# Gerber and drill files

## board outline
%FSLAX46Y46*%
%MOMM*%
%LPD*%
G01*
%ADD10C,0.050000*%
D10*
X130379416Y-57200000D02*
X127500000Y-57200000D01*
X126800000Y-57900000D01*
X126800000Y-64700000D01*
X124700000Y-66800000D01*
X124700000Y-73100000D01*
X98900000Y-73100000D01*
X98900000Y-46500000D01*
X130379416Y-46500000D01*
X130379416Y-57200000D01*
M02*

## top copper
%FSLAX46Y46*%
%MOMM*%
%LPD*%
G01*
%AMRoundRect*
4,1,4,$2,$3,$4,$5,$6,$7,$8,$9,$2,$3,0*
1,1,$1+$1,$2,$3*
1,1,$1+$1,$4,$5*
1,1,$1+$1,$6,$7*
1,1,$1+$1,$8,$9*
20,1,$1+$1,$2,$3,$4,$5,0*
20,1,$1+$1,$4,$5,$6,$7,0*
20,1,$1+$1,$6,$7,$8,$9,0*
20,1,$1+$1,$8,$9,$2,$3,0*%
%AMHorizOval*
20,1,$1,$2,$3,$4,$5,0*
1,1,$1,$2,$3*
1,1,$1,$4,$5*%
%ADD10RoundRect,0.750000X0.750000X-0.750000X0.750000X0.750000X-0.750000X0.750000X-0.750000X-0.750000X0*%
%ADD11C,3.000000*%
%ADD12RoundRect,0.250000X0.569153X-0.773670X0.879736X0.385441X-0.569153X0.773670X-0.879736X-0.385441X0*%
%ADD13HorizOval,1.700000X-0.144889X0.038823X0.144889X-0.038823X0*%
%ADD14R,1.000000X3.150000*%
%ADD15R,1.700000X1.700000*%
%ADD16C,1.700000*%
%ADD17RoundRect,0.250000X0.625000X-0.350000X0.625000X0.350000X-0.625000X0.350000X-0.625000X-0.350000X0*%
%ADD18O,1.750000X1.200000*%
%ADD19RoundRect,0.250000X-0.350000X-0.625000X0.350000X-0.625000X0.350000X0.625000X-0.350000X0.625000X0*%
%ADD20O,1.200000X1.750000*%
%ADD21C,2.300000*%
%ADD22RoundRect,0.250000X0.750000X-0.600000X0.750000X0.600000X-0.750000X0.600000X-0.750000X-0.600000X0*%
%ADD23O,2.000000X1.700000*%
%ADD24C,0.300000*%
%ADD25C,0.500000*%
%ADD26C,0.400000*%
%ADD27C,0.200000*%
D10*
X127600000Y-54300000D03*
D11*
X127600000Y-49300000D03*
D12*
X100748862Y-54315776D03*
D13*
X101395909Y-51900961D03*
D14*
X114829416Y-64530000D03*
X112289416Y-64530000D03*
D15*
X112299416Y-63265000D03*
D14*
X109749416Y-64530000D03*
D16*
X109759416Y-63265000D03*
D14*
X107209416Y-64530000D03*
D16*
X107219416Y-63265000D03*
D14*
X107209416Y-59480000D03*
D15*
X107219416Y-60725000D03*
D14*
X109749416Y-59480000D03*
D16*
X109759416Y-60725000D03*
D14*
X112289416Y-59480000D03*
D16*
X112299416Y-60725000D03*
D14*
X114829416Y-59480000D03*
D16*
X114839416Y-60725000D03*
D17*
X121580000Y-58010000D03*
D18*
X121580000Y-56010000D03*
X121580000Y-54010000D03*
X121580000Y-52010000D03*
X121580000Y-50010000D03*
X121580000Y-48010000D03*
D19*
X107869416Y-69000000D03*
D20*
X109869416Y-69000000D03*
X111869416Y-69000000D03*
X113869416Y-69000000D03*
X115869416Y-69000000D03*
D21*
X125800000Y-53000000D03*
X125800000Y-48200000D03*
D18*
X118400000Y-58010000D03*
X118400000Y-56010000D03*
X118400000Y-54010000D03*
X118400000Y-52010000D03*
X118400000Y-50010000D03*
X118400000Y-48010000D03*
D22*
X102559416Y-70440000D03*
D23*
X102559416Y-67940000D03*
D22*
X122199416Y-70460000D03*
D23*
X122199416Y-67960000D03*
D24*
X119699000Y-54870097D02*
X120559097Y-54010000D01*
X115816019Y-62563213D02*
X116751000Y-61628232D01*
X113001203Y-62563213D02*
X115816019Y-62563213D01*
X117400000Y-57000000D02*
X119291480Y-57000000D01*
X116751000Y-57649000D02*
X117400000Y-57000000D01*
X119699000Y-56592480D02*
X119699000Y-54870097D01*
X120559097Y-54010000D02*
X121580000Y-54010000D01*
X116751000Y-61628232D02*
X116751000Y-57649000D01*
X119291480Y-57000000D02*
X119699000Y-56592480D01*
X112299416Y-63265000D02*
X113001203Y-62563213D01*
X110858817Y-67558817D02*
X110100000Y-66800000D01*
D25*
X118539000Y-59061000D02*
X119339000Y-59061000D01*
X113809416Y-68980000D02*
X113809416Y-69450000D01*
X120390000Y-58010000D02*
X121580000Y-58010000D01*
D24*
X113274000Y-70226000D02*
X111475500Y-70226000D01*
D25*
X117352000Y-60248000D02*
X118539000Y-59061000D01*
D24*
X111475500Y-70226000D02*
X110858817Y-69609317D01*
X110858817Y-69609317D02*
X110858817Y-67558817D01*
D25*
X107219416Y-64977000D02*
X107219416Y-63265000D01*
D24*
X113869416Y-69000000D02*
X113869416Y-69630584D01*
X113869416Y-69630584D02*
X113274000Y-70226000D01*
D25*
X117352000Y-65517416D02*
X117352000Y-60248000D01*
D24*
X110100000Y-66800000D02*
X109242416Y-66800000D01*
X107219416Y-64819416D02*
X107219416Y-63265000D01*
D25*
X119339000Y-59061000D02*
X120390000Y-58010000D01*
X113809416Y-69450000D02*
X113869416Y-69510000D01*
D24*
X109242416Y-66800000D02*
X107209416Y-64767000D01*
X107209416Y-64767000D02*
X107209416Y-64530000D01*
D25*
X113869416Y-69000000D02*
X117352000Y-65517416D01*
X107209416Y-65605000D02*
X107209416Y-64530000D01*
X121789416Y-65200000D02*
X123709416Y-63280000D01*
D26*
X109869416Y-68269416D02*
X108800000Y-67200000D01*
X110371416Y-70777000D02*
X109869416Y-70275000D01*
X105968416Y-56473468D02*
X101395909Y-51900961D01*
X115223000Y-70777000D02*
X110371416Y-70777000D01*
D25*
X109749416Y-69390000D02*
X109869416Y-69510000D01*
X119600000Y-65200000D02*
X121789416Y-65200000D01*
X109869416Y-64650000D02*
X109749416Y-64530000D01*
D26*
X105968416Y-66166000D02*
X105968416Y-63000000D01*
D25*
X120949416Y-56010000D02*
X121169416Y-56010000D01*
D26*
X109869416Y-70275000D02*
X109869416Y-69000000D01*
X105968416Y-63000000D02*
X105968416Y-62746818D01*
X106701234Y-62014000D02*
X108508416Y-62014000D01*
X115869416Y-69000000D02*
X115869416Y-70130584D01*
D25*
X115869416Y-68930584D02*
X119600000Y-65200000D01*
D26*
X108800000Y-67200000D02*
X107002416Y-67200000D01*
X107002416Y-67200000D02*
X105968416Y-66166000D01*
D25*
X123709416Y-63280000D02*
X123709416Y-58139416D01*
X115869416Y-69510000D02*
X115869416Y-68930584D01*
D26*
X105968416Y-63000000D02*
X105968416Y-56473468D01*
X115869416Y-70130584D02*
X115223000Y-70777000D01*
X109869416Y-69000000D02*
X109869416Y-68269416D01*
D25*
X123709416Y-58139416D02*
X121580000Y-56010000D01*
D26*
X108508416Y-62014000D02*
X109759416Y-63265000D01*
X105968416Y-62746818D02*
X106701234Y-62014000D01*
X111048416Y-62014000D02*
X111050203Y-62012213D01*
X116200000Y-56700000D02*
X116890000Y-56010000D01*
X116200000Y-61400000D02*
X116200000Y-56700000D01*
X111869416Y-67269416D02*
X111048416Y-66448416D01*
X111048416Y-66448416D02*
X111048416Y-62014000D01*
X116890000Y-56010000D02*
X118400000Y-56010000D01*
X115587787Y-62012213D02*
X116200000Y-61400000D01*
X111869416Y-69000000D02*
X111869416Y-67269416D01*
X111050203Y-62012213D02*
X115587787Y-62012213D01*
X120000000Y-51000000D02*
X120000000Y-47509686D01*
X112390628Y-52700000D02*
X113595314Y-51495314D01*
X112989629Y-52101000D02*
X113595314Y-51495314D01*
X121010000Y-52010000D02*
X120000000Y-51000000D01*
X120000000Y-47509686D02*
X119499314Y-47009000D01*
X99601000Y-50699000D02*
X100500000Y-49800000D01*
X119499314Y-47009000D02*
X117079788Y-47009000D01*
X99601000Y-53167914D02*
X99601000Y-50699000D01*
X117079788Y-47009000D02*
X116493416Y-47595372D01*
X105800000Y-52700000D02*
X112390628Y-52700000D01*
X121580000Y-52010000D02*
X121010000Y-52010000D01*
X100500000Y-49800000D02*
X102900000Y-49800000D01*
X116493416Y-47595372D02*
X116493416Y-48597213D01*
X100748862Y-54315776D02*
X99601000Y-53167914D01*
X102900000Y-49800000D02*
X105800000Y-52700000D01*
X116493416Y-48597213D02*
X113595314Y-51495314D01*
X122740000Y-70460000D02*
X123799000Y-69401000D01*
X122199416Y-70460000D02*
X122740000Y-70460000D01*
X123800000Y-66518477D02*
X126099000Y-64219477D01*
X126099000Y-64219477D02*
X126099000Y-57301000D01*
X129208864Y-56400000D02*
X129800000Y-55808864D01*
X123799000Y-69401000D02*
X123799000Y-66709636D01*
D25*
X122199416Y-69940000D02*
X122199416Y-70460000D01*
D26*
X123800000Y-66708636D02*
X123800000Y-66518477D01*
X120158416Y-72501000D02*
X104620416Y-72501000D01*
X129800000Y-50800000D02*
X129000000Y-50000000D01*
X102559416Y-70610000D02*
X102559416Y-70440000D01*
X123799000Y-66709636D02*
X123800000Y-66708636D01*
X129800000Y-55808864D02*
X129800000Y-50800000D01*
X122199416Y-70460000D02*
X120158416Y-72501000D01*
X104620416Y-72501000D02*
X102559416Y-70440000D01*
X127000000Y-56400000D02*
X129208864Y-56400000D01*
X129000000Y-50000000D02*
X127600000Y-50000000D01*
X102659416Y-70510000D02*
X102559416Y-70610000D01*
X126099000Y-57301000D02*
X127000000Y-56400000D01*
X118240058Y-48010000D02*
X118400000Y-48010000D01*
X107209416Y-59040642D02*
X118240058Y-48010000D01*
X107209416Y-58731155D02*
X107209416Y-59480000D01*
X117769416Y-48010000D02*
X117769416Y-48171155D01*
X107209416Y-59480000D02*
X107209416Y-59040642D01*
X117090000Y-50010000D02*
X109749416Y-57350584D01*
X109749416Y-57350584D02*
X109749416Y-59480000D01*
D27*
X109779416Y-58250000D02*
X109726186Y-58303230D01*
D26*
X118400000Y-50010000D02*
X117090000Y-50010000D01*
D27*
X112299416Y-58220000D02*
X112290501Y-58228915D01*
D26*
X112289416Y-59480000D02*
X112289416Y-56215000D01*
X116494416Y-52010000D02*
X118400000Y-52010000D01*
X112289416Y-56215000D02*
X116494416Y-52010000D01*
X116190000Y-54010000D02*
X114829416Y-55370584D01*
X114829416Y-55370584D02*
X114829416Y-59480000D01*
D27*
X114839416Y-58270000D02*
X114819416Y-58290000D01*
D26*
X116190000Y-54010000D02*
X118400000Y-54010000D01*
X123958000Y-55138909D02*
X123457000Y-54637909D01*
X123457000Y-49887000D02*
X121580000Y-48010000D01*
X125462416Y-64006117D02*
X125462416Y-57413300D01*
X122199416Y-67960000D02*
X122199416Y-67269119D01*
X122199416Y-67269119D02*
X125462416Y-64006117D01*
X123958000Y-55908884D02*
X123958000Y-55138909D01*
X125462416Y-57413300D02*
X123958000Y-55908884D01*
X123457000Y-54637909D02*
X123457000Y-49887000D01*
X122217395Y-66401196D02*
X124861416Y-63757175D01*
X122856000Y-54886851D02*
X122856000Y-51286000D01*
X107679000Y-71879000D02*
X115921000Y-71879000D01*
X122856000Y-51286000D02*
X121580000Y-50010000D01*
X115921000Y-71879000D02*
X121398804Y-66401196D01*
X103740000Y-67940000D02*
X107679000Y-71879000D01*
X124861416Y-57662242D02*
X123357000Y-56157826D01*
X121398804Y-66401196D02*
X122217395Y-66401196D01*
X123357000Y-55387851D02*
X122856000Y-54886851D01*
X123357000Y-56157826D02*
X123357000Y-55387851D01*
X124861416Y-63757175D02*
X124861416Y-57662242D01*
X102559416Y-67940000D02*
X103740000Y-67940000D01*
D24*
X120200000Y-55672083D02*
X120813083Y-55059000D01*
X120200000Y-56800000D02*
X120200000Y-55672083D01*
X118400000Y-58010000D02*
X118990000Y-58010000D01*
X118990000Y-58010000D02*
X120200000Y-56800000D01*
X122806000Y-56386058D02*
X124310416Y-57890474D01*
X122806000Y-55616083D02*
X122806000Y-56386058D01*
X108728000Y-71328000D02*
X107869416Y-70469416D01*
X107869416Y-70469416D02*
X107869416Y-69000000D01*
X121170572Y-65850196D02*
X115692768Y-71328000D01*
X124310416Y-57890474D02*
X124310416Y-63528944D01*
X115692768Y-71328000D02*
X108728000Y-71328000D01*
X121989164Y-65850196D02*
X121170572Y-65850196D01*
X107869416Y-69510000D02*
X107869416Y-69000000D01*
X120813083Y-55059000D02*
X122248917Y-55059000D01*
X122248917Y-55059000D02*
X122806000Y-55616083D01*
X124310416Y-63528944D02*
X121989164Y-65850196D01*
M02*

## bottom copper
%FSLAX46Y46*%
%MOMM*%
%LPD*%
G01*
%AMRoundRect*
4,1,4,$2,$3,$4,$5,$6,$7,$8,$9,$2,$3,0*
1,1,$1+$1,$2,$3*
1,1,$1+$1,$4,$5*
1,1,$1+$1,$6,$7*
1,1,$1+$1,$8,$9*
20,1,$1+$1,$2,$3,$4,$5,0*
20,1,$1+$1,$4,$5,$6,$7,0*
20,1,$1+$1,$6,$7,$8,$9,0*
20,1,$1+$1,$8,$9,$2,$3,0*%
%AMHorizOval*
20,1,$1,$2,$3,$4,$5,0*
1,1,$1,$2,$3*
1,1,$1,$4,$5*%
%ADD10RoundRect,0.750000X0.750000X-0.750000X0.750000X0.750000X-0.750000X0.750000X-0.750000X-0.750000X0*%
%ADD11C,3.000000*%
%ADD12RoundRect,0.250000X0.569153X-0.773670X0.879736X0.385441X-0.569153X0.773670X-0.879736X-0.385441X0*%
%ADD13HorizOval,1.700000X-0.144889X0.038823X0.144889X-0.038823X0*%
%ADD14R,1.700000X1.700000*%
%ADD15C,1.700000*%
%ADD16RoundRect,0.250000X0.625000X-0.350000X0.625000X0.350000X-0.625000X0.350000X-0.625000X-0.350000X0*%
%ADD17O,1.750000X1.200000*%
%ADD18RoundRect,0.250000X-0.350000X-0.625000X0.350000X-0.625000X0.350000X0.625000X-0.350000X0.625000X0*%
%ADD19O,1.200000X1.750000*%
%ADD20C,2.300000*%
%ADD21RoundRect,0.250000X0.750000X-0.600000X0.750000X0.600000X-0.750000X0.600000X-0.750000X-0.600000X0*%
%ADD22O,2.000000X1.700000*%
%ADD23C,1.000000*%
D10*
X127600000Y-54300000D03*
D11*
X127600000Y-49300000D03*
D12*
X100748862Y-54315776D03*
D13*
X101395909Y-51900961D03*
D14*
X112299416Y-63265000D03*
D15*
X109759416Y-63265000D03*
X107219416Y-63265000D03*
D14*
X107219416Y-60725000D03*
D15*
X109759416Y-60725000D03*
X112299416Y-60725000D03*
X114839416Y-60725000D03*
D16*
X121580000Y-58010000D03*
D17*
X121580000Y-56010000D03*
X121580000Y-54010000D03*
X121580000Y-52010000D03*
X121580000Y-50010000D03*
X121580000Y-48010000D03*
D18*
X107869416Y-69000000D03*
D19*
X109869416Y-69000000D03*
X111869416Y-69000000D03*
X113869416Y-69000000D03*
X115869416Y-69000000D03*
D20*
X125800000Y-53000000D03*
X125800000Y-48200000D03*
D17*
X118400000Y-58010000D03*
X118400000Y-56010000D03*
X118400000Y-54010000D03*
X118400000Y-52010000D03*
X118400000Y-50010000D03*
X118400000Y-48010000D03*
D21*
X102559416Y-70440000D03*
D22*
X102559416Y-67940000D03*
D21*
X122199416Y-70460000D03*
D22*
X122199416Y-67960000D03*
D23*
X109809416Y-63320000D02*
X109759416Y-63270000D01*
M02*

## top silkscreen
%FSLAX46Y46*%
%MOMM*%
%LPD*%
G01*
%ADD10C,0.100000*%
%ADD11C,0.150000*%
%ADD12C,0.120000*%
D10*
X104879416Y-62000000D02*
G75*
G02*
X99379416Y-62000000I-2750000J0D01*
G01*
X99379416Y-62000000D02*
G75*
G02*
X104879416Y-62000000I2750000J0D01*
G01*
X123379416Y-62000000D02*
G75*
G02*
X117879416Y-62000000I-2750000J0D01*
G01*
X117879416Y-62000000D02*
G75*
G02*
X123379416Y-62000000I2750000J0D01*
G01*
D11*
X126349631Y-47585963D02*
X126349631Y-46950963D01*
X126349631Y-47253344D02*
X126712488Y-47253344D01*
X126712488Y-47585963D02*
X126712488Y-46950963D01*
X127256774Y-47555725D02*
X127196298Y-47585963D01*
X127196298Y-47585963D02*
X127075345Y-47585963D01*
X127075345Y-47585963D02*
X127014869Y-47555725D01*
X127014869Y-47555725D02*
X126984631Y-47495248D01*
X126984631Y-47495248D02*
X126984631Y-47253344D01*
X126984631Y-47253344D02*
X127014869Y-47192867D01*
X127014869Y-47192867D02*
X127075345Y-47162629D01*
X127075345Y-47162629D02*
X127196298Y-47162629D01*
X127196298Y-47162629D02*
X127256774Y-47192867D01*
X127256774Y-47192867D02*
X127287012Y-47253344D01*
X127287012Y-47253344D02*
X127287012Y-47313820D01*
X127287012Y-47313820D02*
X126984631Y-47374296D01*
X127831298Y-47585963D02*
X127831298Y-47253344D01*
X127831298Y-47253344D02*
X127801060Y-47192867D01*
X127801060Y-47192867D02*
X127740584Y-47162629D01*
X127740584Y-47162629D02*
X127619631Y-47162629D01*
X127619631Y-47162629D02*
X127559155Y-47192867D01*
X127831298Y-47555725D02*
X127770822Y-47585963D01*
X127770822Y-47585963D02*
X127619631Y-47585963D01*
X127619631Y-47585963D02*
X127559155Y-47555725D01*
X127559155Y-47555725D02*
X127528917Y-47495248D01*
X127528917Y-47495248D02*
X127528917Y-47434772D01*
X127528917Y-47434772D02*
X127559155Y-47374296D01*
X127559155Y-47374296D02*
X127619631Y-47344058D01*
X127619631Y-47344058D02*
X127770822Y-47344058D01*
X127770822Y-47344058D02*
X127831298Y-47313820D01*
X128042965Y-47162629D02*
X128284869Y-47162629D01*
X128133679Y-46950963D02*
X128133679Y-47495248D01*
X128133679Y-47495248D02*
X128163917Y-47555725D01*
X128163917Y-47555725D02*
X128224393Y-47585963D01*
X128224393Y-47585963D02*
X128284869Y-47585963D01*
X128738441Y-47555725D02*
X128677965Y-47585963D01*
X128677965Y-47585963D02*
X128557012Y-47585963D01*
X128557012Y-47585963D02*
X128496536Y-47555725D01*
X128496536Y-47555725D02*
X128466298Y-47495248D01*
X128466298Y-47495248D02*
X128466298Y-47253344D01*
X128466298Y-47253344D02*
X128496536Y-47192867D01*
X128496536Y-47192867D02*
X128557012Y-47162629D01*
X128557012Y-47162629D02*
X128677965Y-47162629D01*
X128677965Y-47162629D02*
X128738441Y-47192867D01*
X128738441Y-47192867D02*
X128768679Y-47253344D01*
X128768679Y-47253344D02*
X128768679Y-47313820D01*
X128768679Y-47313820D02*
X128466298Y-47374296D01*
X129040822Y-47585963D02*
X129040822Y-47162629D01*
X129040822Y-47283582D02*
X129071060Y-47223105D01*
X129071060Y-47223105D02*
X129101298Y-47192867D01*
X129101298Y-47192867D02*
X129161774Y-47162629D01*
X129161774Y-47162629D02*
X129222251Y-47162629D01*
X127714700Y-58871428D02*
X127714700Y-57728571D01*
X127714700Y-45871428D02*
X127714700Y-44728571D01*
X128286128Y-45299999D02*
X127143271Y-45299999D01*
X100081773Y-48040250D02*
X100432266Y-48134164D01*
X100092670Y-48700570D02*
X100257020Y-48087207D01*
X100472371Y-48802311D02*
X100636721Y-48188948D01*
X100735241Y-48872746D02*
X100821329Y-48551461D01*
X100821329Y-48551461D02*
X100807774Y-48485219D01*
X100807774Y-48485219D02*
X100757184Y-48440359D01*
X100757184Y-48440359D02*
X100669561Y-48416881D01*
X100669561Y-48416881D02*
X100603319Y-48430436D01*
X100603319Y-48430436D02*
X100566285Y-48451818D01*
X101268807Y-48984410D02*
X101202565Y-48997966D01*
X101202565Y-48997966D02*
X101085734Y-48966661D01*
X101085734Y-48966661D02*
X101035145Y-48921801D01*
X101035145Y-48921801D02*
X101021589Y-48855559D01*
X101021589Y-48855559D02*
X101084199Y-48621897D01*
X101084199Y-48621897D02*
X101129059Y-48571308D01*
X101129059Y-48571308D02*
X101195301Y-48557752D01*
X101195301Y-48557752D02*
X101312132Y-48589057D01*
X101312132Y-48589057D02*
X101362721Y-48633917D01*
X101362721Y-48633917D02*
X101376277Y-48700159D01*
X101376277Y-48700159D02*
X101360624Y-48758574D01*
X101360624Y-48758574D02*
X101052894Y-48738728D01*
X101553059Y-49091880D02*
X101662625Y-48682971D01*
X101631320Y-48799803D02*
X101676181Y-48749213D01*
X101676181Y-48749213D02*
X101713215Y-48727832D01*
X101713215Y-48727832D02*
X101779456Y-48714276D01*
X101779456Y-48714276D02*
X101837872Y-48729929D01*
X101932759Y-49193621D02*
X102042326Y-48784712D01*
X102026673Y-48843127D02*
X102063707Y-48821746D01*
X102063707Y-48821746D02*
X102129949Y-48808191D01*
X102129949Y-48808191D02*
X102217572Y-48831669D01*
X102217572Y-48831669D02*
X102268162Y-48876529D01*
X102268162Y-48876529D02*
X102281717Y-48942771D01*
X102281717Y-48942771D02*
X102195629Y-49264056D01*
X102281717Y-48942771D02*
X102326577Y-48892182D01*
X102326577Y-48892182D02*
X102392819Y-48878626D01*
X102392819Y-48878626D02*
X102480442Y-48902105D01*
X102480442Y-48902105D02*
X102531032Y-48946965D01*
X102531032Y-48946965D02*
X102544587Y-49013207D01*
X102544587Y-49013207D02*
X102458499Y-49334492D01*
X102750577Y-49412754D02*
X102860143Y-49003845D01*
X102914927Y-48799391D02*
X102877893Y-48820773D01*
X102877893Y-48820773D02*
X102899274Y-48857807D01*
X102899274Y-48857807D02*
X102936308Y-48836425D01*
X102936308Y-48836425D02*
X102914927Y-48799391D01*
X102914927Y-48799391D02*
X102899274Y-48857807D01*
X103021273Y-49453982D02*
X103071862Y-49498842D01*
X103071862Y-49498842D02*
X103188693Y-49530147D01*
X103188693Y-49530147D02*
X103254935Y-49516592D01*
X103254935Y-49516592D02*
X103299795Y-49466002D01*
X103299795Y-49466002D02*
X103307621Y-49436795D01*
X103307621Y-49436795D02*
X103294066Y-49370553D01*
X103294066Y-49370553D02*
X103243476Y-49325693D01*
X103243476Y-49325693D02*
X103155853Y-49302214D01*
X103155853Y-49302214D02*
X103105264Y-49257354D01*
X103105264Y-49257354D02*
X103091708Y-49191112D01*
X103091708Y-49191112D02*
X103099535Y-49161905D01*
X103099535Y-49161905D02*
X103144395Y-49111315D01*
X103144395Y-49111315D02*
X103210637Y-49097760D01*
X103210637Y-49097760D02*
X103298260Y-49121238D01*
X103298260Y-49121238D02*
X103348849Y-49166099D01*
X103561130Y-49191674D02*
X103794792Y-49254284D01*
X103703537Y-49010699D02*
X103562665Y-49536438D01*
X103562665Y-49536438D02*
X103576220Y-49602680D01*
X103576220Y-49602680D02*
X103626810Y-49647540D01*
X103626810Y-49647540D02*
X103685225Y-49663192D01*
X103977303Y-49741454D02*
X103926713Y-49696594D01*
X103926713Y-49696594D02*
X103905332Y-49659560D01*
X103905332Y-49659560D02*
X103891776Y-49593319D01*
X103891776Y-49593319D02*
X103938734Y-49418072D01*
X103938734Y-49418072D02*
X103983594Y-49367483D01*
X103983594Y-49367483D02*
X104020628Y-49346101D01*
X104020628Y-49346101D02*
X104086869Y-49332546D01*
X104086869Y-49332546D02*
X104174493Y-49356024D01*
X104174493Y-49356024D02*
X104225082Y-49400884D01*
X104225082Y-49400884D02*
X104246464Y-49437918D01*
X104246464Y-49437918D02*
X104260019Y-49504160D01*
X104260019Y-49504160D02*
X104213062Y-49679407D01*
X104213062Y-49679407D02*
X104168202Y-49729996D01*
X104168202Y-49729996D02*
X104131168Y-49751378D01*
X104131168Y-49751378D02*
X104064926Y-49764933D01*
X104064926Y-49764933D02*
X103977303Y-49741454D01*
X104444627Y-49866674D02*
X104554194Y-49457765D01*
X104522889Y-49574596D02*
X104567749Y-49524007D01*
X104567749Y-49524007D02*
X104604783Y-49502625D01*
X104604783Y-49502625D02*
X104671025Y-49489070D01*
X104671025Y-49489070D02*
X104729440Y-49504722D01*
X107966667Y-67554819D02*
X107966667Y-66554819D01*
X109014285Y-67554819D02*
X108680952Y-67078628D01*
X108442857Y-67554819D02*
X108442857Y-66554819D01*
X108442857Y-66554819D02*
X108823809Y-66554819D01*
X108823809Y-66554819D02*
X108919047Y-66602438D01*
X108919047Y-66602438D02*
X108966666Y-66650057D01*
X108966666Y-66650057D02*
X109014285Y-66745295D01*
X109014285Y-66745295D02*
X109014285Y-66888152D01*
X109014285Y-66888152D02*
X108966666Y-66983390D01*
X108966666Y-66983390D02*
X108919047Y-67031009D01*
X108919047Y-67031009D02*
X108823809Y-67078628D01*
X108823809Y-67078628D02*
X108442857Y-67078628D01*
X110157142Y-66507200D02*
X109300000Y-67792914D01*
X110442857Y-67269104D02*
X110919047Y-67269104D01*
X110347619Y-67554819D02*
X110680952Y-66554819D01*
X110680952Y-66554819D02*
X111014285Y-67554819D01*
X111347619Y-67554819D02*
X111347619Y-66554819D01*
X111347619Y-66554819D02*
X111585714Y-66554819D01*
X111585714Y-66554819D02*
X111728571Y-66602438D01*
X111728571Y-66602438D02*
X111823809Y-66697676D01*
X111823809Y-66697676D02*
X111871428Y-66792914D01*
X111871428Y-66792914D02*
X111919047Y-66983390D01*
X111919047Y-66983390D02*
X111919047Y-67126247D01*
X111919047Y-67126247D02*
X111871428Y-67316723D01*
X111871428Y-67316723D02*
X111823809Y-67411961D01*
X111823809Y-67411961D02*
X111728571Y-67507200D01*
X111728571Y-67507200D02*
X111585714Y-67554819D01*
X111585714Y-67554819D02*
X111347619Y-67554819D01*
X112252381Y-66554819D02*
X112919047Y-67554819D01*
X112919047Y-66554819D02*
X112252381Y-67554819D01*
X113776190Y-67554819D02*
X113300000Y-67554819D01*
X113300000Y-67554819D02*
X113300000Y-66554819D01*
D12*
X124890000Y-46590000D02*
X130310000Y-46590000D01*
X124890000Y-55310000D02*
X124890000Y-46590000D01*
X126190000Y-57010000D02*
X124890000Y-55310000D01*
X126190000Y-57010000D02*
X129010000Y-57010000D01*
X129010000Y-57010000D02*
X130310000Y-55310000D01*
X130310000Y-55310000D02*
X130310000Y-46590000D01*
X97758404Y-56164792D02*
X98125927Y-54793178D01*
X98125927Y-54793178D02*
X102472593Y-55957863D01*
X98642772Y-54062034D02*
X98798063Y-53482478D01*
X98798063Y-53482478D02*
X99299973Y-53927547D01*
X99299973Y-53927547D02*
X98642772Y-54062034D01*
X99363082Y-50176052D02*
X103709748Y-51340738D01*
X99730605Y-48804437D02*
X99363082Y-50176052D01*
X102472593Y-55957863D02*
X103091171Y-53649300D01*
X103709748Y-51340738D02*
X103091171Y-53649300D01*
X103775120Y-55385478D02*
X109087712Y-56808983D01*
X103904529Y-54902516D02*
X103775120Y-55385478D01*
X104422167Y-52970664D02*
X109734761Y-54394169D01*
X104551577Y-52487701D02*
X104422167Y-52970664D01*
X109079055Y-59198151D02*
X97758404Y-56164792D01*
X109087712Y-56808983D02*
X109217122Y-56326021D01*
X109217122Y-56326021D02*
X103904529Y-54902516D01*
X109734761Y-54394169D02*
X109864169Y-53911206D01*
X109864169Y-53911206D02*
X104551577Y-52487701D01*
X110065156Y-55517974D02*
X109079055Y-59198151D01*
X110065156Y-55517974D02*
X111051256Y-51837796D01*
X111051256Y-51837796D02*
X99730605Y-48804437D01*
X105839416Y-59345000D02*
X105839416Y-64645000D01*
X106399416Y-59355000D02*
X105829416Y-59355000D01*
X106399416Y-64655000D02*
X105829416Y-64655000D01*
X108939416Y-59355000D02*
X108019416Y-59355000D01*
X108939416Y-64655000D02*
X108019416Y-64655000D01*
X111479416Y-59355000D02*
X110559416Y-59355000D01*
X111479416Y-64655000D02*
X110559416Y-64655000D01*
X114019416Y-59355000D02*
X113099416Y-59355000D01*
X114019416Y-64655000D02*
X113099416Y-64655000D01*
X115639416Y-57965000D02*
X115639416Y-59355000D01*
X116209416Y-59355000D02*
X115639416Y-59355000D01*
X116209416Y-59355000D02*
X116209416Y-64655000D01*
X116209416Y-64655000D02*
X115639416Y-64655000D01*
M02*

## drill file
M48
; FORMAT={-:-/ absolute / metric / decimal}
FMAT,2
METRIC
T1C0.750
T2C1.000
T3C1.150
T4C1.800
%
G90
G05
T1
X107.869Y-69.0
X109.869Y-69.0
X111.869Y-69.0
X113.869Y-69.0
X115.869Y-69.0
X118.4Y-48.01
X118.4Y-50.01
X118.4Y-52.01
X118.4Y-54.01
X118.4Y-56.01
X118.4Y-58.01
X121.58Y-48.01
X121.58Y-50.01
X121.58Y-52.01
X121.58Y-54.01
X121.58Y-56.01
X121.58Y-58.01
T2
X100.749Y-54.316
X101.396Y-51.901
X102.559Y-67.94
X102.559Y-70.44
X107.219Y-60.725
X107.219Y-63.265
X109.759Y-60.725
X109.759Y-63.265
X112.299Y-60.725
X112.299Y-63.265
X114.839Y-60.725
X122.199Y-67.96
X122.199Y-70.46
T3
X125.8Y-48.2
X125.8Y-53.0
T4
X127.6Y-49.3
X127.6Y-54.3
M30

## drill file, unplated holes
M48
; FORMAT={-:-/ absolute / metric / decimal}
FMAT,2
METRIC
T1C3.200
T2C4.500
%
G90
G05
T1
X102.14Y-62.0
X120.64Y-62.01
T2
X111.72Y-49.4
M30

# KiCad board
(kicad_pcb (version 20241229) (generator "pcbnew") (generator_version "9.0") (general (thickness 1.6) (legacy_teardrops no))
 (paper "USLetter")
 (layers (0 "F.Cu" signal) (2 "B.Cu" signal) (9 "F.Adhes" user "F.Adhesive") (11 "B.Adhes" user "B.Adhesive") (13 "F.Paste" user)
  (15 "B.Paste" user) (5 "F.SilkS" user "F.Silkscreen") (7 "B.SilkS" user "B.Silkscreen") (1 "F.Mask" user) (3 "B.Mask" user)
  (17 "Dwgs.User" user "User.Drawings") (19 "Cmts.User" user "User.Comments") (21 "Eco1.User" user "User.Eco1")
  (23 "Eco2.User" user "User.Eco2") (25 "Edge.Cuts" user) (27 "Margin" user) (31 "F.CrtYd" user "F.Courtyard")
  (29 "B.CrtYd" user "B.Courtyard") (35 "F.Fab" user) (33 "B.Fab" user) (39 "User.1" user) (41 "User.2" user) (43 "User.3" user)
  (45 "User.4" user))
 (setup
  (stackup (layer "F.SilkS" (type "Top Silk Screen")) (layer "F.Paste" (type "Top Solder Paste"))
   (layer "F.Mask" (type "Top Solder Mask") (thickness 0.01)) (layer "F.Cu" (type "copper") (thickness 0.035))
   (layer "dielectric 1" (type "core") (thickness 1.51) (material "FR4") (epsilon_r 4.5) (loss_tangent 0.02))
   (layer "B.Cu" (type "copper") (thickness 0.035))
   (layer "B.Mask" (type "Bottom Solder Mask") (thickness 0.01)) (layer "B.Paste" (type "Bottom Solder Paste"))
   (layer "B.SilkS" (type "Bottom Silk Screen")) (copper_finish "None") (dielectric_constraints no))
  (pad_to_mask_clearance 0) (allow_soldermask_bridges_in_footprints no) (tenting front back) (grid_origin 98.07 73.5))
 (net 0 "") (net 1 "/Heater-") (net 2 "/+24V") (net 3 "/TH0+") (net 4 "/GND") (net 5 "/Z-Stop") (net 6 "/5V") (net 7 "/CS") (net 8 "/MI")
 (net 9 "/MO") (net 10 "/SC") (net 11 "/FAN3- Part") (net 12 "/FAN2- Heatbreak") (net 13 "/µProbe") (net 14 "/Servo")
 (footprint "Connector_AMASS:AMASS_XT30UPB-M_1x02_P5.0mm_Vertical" (layer "F.Cu") (at 127.6 54.3 90)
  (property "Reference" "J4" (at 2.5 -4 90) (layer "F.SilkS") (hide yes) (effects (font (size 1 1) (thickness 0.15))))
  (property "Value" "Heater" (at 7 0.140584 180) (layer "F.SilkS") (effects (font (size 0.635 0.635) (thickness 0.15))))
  (fp_line (start 7.71 -2.71) (end 7.71 2.71) (stroke (width 0.12) (type solid)) (layer "F.SilkS"))
  (fp_line (start -1.01 -2.71) (end 7.71 -2.71) (stroke (width 0.12) (type solid)) (layer "F.SilkS"))
  (fp_line (start -2.71 -1.41) (end -1.01 -2.71) (stroke (width 0.12) (type solid)) (layer "F.SilkS"))
  (fp_line (start -2.71 -1.41) (end -2.71 1.41) (stroke (width 0.12) (type solid)) (layer "F.SilkS"))
  (fp_line (start -2.71 1.41) (end -1.01 2.71) (stroke (width 0.12) (type solid)) (layer "F.SilkS"))
  (fp_line (start -1.01 2.71) (end 7.71 2.71) (stroke (width 0.12) (type solid)) (layer "F.SilkS"))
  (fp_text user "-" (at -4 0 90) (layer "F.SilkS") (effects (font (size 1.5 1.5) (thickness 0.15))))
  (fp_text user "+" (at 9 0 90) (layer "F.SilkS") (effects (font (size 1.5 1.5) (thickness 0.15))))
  (pad "1" thru_hole roundrect (at 0 0 90) (size 3 3) (drill 1.8) (layers "*.Cu" "*.Mask") (remove_unused_layers no) (roundrect_rratio 0.25)
   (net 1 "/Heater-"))
  (pad "2" thru_hole circle (at 5 0 90) (size 3 3) (drill 1.8) (layers "*.Cu" "*.Mask") (remove_unused_layers no) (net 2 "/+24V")))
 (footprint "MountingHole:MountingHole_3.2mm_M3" (layer "F.Cu") (at 120.64 62.01)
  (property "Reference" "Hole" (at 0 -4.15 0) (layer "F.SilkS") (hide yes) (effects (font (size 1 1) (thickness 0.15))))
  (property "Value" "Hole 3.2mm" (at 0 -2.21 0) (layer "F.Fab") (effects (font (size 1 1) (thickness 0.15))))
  (pad "" np_thru_hole circle (at 0 0) (size 3.2 3.2) (drill 3.2) (layers "*.Cu" "*.Mask")))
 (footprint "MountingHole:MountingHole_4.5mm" (layer "F.Cu") (at 111.72 49.4)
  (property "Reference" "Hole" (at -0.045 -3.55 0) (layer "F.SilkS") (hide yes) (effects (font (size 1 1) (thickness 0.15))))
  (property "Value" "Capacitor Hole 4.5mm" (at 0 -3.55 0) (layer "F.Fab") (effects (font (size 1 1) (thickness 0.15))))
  (pad "" np_thru_hole circle (at 0 0) (size 4.5 4.5) (drill 4.5) (layers "*.Cu" "*.Mask")))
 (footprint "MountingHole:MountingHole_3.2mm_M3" (layer "F.Cu") (at 102.14 62)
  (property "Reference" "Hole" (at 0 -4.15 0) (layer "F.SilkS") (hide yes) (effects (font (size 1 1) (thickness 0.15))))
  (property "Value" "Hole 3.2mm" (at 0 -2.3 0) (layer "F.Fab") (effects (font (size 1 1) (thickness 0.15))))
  (pad "" np_thru_hole circle (at 0 0) (size 3.2 3.2) (drill 3.2) (layers "*.Cu" "*.Mask")))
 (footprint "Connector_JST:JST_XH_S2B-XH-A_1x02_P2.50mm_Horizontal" (layer "F.Cu") (at 100.748862 54.315776 75)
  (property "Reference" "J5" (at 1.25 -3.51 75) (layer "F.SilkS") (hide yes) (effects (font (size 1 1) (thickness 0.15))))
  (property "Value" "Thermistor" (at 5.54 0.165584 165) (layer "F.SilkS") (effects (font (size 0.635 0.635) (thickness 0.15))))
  (fp_line (start -2.56 -2.41) (end -1.14 -2.41) (stroke (width 0.12) (type solid)) (layer "F.SilkS"))
  (fp_line (start -1.14 -2.41) (end -1.14 2.09) (stroke (width 0.12) (type solid)) (layer "F.SilkS"))
  (fp_line (start -0.3 -2.1) (end 0.3 -2.100001) (stroke (width 0.12) (type solid)) (layer "F.SilkS"))
  (fp_line (start 0.3 -2.100001) (end 0 -1.5) (stroke (width 0.12) (type solid)) (layer "F.SilkS"))
  (fp_line (start 0 -1.5) (end -0.3 -2.1) (stroke (width 0.12) (type solid)) (layer "F.SilkS"))
  (fp_line (start 3.64 -2.41) (end 3.64 2.09) (stroke (width 0.12) (type solid)) (layer "F.SilkS"))
  (fp_line (start 5.06 -2.41) (end 3.64 -2.41) (stroke (width 0.12) (type solid)) (layer "F.SilkS"))
  (fp_line (start -1.14 2.09) (end 1.250001 2.09) (stroke (width 0.12) (type solid)) (layer "F.SilkS"))
  (fp_line (start 3.64 2.09) (end 1.250001 2.09) (stroke (width 0.12) (type solid)) (layer "F.SilkS"))
  (fp_line (start -0.25 3.2) (end -0.25 8.7) (stroke (width 0.12) (type solid)) (layer "F.SilkS"))
  (fp_line (start 0.249999 3.2) (end -0.25 3.2) (stroke (width 0.12) (type solid)) (layer "F.SilkS"))
  (fp_line (start 2.25 3.2) (end 2.25 8.700002) (stroke (width 0.12) (type solid)) (layer "F.SilkS"))
  (fp_line (start 2.75 3.2) (end 2.25 3.2) (stroke (width 0.12) (type solid)) (layer "F.SilkS"))
  (fp_line (start -2.56 9.31) (end -2.56 -2.41) (stroke (width 0.12) (type solid)) (layer "F.SilkS"))
  (fp_line (start -0.25 8.7) (end 0.249999 8.700001) (stroke (width 0.12) (type solid)) (layer "F.SilkS"))
  (fp_line (start 0.249999 8.700001) (end 0.249999 3.2) (stroke (width 0.12) (type solid)) (layer "F.SilkS"))
  (fp_line (start 2.25 8.700002) (end 2.75 8.7) (stroke (width 0.12) (type solid)) (layer "F.SilkS"))
  (fp_line (start 2.75 8.7) (end 2.75 3.2) (stroke (width 0.12) (type solid)) (layer "F.SilkS"))
  (fp_line (start 1.25 9.310001) (end -2.56 9.31) (stroke (width 0.12) (type solid)) (layer "F.SilkS"))
  (fp_line (start 1.25 9.310001) (end 5.060001 9.31) (stroke (width 0.12) (type solid)) (layer "F.SilkS"))
  (fp_line (start 5.060001 9.31) (end 5.06 -2.41) (stroke (width 0.12) (type solid)) (layer "F.SilkS"))
  (pad "1" thru_hole roundrect (at 0 0 75) (size 1.7 2) (drill 1) (layers "*.Cu" "*.Mask") (remove_unused_layers no)
   (roundrect_rratio 0.147059) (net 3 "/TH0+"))
  (pad "2" thru_hole oval (at 2.5 -0.000001 75) (size 1.7 2) (drill 1) (layers "*.Cu" "*.Mask") (remove_unused_layers no) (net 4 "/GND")))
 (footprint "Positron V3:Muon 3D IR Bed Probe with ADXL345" (layer "F.Cu") (at 109.339416 58.225)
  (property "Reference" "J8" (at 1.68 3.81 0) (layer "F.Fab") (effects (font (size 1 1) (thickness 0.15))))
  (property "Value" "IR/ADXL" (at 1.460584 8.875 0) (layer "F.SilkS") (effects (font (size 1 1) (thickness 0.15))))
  (fp_line (start -3.5 1.12) (end -3.5 6.42) (stroke (width 0.12) (type solid)) (layer "F.SilkS"))
  (fp_line (start -2.94 1.13) (end -3.51 1.13) (stroke (width 0.12) (type solid)) (layer "F.SilkS"))
  (fp_line (start -2.94 6.43) (end -3.51 6.43) (stroke (width 0.12) (type solid)) (layer "F.SilkS"))
  (fp_line (start -0.4 1.13) (end -1.32 1.13) (stroke (width 0.12) (type solid)) (layer "F.SilkS"))
  (fp_line (start -0.4 6.43) (end -1.32 6.43) (stroke (width 0.12) (type solid)) (layer "F.SilkS"))
  (fp_line (start 2.14 1.13) (end 1.22 1.13) (stroke (width 0.12) (type solid)) (layer "F.SilkS"))
  (fp_line (start 2.14 6.43) (end 1.22 6.43) (stroke (width 0.12) (type solid)) (layer "F.SilkS"))
  (fp_line (start 4.68 1.13) (end 3.76 1.13) (stroke (width 0.12) (type solid)) (layer "F.SilkS"))
  (fp_line (start 4.68 6.43) (end 3.76 6.43) (stroke (width 0.12) (type solid)) (layer "F.SilkS"))
  (fp_line (start 6.3 -0.26) (end 6.3 1.13) (stroke (width 0.12) (type solid)) (layer "F.SilkS"))
  (fp_line (start 6.87 1.13) (end 6.3 1.13) (stroke (width 0.12) (type solid)) (layer "F.SilkS"))
  (fp_line (start 6.87 1.13) (end 6.87 6.43) (stroke (width 0.12) (type solid)) (layer "F.SilkS"))
  (fp_line (start 6.87 6.43) (end 6.3 6.43) (stroke (width 0.12) (type solid)) (layer "F.SilkS"))
  (pad "" smd rect (at 5.49 6.305 270) (size 3.15 1) (layers "F.Cu" "F.Mask" "F.Paste"))
  (pad "1" smd rect (at 2.95 6.305 270) (size 3.15 1) (layers "F.Cu" "F.Mask" "F.Paste") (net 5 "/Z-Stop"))
  (pad "1" thru_hole rect (at 2.96 5.04 270) (size 1.7 1.7) (drill 1) (layers "*.Cu" "*.Mask") (remove_unused_layers no) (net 5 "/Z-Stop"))
  (pad "2" smd rect (at 0.41 6.305 270) (size 3.15 1) (layers "F.Cu" "F.Mask" "F.Paste") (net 4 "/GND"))
  (pad "2" thru_hole circle (at 0.42 5.04 270) (size 1.7 1.7) (drill 1) (layers "*.Cu" "*.Mask") (remove_unused_layers no) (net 4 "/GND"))
  (pad "3" smd rect (at -2.13 6.305 270) (size 3.15 1) (layers "F.Cu" "F.Mask" "F.Paste") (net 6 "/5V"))
  (pad "3" thru_hole circle (at -2.12 5.04 270) (size 1.7 1.7) (drill 1) (layers "*.Cu" "*.Mask") (remove_unused_layers no) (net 6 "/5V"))
  (pad "4" smd rect (at -2.13 1.255 270) (size 3.15 1) (layers "F.Cu" "F.Mask" "F.Paste") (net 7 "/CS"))
  (pad "4" thru_hole rect (at -2.12 2.5 270) (size 1.7 1.7) (drill 1) (layers "*.Cu" "*.Mask") (remove_unused_layers no) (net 7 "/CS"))
  (pad "5" smd rect (at 0.41 1.255 270) (size 3.15 1) (layers "F.Cu" "F.Mask" "F.Paste") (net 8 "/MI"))
  (pad "5" thru_hole circle (at 0.42 2.5 270) (size 1.7 1.7) (drill 1) (layers "*.Cu" "*.Mask") (remove_unused_layers no) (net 8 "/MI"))
  (pad "6" smd rect (at 2.95 1.255 270) (size 3.15 1) (layers "F.Cu" "F.Mask" "F.Paste") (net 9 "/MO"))
  (pad "6" thru_hole circle (at 2.96 2.5 270) (size 1.7 1.7) (drill 1) (layers "*.Cu" "*.Mask") (remove_unused_layers no) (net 9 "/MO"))
  (pad "7" smd rect (at 5.49 1.255 270) (size 3.15 1) (layers "F.Cu" "F.Mask" "F.Paste") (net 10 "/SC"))
  (pad "7" thru_hole circle (at 5.5 2.5 270) (size 1.7 1.7) (drill 1) (layers "*.Cu" "*.Mask") (remove_unused_layers no) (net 10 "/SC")))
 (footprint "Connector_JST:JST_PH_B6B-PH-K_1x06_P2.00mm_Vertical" (layer "B.Cu") (at 121.58 58.01 90)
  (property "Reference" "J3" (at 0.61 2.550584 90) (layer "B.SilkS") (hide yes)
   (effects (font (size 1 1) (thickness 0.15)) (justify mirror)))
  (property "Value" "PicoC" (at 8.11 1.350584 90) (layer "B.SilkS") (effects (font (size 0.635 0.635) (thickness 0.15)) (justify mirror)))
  (pad "1" thru_hole roundrect (at 0 0 90) (size 1.2 1.75) (drill 0.75) (layers "*.Cu" "*.Mask") (remove_unused_layers no)
   (roundrect_rratio 0.208333) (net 6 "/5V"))
  (pad "2" thru_hole oval (at 2 0 90) (size 1.2 1.75) (drill 0.75) (layers "*.Cu" "*.Mask") (remove_unused_layers no) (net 4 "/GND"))
  (pad "3" thru_hole oval (at 4 0 90) (size 1.2 1.75) (drill 0.75) (layers "*.Cu" "*.Mask") (remove_unused_layers no) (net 5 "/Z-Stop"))
  (pad "4" thru_hole oval (at 6 0 90) (size 1.2 1.75) (drill 0.75) (layers "*.Cu" "*.Mask") (remove_unused_layers no) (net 3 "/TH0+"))
  (pad "5" thru_hole oval (at 8 0 90) (size 1.2 1.75) (drill 0.75) (layers "*.Cu" "*.Mask") (remove_unused_layers no) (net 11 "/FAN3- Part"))
  (pad "6" thru_hole oval (at 10 0 90) (size 1.2 1.75) (drill 0.75) (layers "*.Cu" "*.Mask") (remove_unused_layers no)
   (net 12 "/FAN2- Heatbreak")))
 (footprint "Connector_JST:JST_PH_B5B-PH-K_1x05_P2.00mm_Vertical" (layer "B.Cu") (at 107.869416 69)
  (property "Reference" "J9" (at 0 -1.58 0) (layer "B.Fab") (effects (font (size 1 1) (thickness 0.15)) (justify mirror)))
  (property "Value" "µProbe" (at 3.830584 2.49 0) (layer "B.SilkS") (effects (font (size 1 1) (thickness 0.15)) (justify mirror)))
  (pad "1" thru_hole roundrect (at 0 0) (size 1.2 1.75) (drill 0.75) (layers "*.Cu" "*.Mask") (remove_unused_layers no)
   (roundrect_rratio 0.208333) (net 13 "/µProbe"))
  (pad "2" thru_hole oval (at 2 0) (size 1.2 1.75) (drill 0.75) (layers "*.Cu" "*.Mask") (remove_unused_layers no) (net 4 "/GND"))
  (pad "3" thru_hole oval (at 4 0) (size 1.2 1.75) (drill 0.75) (layers "*.Cu" "*.Mask") (remove_unused_layers no) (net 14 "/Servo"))
  (pad "4" thru_hole oval (at 6 0) (size 1.2 1.75) (drill 0.75) (layers "*.Cu" "*.Mask") (remove_unused_layers no) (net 6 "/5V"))
  (pad "5" thru_hole oval (at 8 0) (size 1.2 1.75) (drill 0.75) (layers "*.Cu" "*.Mask") (remove_unused_layers no) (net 4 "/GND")))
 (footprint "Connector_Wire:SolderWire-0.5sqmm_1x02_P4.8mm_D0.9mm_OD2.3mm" (layer "B.Cu") (at 125.8 53 90)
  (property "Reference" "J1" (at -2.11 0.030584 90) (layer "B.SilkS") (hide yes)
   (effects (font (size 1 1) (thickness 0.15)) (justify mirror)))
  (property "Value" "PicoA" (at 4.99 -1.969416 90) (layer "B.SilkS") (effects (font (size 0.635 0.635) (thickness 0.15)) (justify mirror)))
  (pad "1" thru_hole circle (at 0 0 90) (size 2.3 2.3) (drill 1.15) (layers "*.Cu" "*.Mask") (remove_unused_layers no) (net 1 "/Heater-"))
  (pad "2" thru_hole circle (at 4.8 0 90) (size 2.3 2.3) (drill 1.15) (layers "*.Cu" "*.Mask") (remove_unused_layers no) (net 2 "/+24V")))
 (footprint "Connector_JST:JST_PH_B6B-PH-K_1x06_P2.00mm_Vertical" (layer "B.Cu") (at 118.4 58.01 90)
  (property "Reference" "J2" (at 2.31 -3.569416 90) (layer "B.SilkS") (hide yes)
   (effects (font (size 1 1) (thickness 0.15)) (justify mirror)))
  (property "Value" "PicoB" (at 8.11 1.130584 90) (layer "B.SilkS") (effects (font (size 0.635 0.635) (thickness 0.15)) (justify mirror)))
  (pad "1" thru_hole oval (at 0 0 90) (size 1.2 1.75) (drill 0.75) (layers "*.Cu" "*.Mask") (remove_unused_layers no) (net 13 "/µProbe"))
  (pad "2" thru_hole oval (at 2 0 90) (size 1.2 1.75) (drill 0.75) (layers "*.Cu" "*.Mask") (remove_unused_layers no) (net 14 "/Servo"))
  (pad "3" thru_hole oval (at 4 0 90) (size 1.2 1.75) (drill 0.75) (layers "*.Cu" "*.Mask") (remove_unused_layers no) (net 10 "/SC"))
  (pad "4" thru_hole oval (at 6 0 90) (size 1.2 1.75) (drill 0.75) (layers "*.Cu" "*.Mask") (remove_unused_layers no) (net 9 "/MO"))
  (pad "5" thru_hole oval (at 8 0 90) (size 1.2 1.75) (drill 0.75) (layers "*.Cu" "*.Mask") (remove_unused_layers no) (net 8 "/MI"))
  (pad "6" thru_hole oval (at 10 0 90) (size 1.2 1.75) (drill 0.75) (layers "*.Cu" "*.Mask") (remove_unused_layers no) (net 7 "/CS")))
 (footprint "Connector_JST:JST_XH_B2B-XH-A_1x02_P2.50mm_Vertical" (layer "B.Cu") (at 102.559416 70.44 90)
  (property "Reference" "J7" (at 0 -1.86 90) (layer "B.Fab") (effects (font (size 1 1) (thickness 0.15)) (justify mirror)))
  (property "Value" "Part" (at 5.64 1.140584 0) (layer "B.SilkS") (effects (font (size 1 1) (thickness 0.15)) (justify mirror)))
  (pad "1" thru_hole roundrect (at 0 0 90) (size 1.7 2) (drill 1) (layers "*.Cu" "*.Mask") (remove_unused_layers no)
   (roundrect_rratio 0.147059) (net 2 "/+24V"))
  (pad "2" thru_hole oval (at 2.5 0 90) (size 1.7 2) (drill 1) (layers "*.Cu" "*.Mask") (remove_unused_layers no) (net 11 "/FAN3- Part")))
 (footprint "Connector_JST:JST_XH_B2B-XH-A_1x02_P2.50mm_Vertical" (layer "B.Cu") (at 122.199416 70.46 90)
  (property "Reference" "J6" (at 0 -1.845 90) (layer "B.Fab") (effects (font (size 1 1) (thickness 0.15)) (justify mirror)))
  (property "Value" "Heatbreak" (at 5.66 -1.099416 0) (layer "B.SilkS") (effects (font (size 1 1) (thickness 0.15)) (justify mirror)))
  (pad "1" thru_hole roundrect (at 0 0 90) (size 1.7 2) (drill 1) (layers "*.Cu" "*.Mask") (remove_unused_layers no)
   (roundrect_rratio 0.147059) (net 2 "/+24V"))
  (pad "2" thru_hole oval (at 2.5 0 90) (size 1.7 2) (drill 1) (layers "*.Cu" "*.Mask") (remove_unused_layers no)
   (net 12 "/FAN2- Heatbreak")))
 (gr_circle (center 102.129416 62) (end 104.879416 62) (stroke (width 0.1) (type solid)) (fill no) (layer "F.SilkS"))
 (gr_circle (center 120.629416 62) (end 123.379416 62) (stroke (width 0.1) (type solid)) (fill no) (layer "F.SilkS"))
 (gr_poly
  (pts (xy 130.379416 46.5) (xy 130.379416 57.2) (xy 127.5 57.2) (xy 126.8 57.9) (xy 126.8 64.7) (xy 124.7 66.8) (xy 124.7 73.1)
   (xy 98.9 73.1) (xy 98.9 46.5))
  (stroke (width 0.05) (type solid)) (fill no) (layer "Edge.Cuts"))
 (segment (start 119.699 54.870097) (end 120.559097 54.01) (width 0.3) (layer "F.Cu") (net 5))
 (segment (start 115.816019 62.563213) (end 116.751 61.628232) (width 0.3) (layer "F.Cu") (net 5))
 (segment (start 113.001203 62.563213) (end 115.816019 62.563213) (width 0.3) (layer "F.Cu") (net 5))
 (segment (start 117.4 57) (end 119.29148 57) (width 0.3) (layer "F.Cu") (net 5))
 (segment (start 116.751 57.649) (end 117.4 57) (width 0.3) (layer "F.Cu") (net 5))
 (segment (start 119.699 56.59248) (end 119.699 54.870097) (width 0.3) (layer "F.Cu") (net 5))
 (segment (start 120.559097 54.01) (end 121.58 54.01) (width 0.3) (layer "F.Cu") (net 5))
 (segment (start 116.751 61.628232) (end 116.751 57.649) (width 0.3) (layer "F.Cu") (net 5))
 (segment (start 119.29148 57) (end 119.699 56.59248) (width 0.3) (layer "F.Cu") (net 5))
 (segment (start 112.299416 63.265) (end 113.001203 62.563213) (width 0.3) (layer "F.Cu") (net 5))
 (segment (start 110.858817 67.558817) (end 110.1 66.8) (width 0.3) (layer "F.Cu") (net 6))
 (segment (start 118.539 59.061) (end 119.339 59.061) (width 0.5) (layer "F.Cu") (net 6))
 (segment (start 113.809416 68.98) (end 113.809416 69.45) (width 0.5) (layer "F.Cu") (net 6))
 (segment (start 120.39 58.01) (end 121.58 58.01) (width 0.5) (layer "F.Cu") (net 6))
 (segment (start 113.274 70.226) (end 111.4755 70.226) (width 0.3) (layer "F.Cu") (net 6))
 (segment (start 117.352 60.248) (end 118.539 59.061) (width 0.5) (layer "F.Cu") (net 6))
 (segment (start 111.4755 70.226) (end 110.858817 69.609317) (width 0.3) (layer "F.Cu") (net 6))
 (segment (start 110.858817 69.609317) (end 110.858817 67.558817) (width 0.3) (layer "F.Cu") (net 6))
 (segment (start 107.219416 64.977) (end 107.219416 63.265) (width 0.5) (layer "F.Cu") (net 6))
 (segment (start 113.869416 69) (end 113.869416 69.630584) (width 0.3) (layer "F.Cu") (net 6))
 (segment (start 113.869416 69.630584) (end 113.274 70.226) (width 0.3) (layer "F.Cu") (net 6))
 (segment (start 117.352 65.517416) (end 117.352 60.248) (width 0.5) (layer "F.Cu") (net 6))
 (segment (start 110.1 66.8) (end 109.242416 66.8) (width 0.3) (layer "F.Cu") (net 6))
 (segment (start 107.219416 64.819416) (end 107.219416 63.265) (width 0.3) (layer "F.Cu") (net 6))
 (segment (start 119.339 59.061) (end 120.39 58.01) (width 0.5) (layer "F.Cu") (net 6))
 (segment (start 113.809416 69.45) (end 113.869416 69.51) (width 0.5) (layer "F.Cu") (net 6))
 (segment (start 109.242416 66.8) (end 107.209416 64.767) (width 0.3) (layer "F.Cu") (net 6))
 (segment (start 107.209416 64.767) (end 107.209416 64.53) (width 0.3) (layer "F.Cu") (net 6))
 (segment (start 113.869416 69) (end 117.352 65.517416) (width 0.5) (layer "F.Cu") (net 6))
 (segment (start 107.209416 65.605) (end 107.209416 64.53) (width 0.5) (layer "F.Cu") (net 6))
 (segment (start 121.789416 65.2) (end 123.709416 63.28) (width 0.5) (layer "F.Cu") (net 4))
 (segment (start 109.869416 68.269416) (end 108.8 67.2) (width 0.4) (layer "F.Cu") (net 4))
 (segment (start 110.371416 70.777) (end 109.869416 70.275) (width 0.4) (layer "F.Cu") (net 4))
 (segment (start 105.968416 56.473468) (end 101.395909 51.900961) (width 0.4) (layer "F.Cu") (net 4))
 (segment (start 115.223 70.777) (end 110.371416 70.777) (width 0.4) (layer "F.Cu") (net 4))
 (segment (start 109.749416 69.39) (end 109.869416 69.51) (width 0.5) (layer "F.Cu") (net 4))
 (segment (start 119.6 65.2) (end 121.789416 65.2) (width 0.5) (layer "F.Cu") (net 4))
 (segment (start 109.869416 64.65) (end 109.749416 64.53) (width 0.5) (layer "F.Cu") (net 4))
 (segment (start 105.968416 66.166) (end 105.968416 63) (width 0.4) (layer "F.Cu") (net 4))
 (segment (start 120.949416 56.01) (end 121.169416 56.01) (width 0.5) (layer "F.Cu") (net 4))
 (segment (start 109.869416 70.275) (end 109.869416 69) (width 0.4) (layer "F.Cu") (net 4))
 (segment (start 105.968416 63) (end 105.968416 62.746818) (width 0.4) (layer "F.Cu") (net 4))
 (segment (start 106.701234 62.014) (end 108.508416 62.014) (width 0.4) (layer "F.Cu") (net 4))
 (segment (start 115.869416 69) (end 115.869416 70.130584) (width 0.4) (layer "F.Cu") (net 4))
 (segment (start 115.869416 68.930584) (end 119.6 65.2) (width 0.5) (layer "F.Cu") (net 4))
 (segment (start 108.8 67.2) (end 107.002416 67.2) (width 0.4) (layer "F.Cu") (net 4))
 (segment (start 107.002416 67.2) (end 105.968416 66.166) (width 0.4) (layer "F.Cu") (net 4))
 (segment (start 123.709416 63.28) (end 123.709416 58.139416) (width 0.5) (layer "F.Cu") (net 4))
 (segment (start 115.869416 69.51) (end 115.869416 68.930584) (width 0.5) (layer "F.Cu") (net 4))
 (segment (start 105.968416 63) (end 105.968416 56.473468) (width 0.4) (layer "F.Cu") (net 4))
 (segment (start 115.869416 70.130584) (end 115.223 70.777) (width 0.4) (layer "F.Cu") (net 4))
 (segment (start 109.869416 69) (end 109.869416 68.269416) (width 0.4) (layer "F.Cu") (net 4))
 (segment (start 123.709416 58.139416) (end 121.58 56.01) (width 0.5) (layer "F.Cu") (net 4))
 (segment (start 108.508416 62.014) (end 109.759416 63.265) (width 0.4) (layer "F.Cu") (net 4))
 (segment (start 105.968416 62.746818) (end 106.701234 62.014) (width 0.4) (layer "F.Cu") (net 4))
 (segment (start 109.809416 63.32) (end 109.759416 63.27) (width 1) (layer "B.Cu") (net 4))
 (segment (start 111.048416 62.014) (end 111.050203 62.012213) (width 0.4) (layer "F.Cu") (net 14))
 (segment (start 116.2 56.7) (end 116.89 56.01) (width 0.4) (layer "F.Cu") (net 14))
 (segment (start 116.2 61.4) (end 116.2 56.7) (width 0.4) (layer "F.Cu") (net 14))
 (segment (start 111.869416 67.269416) (end 111.048416 66.448416) (width 0.4) (layer "F.Cu") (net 14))
 (segment (start 111.048416 66.448416) (end 111.048416 62.014) (width 0.4) (layer "F.Cu") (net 14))
 (segment (start 116.89 56.01) (end 118.4 56.01) (width 0.4) (layer "F.Cu") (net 14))
 (segment (start 115.587787 62.012213) (end 116.2 61.4) (width 0.4) (layer "F.Cu") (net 14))
 (segment (start 111.869416 69) (end 111.869416 67.269416) (width 0.4) (layer "F.Cu") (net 14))
 (segment (start 111.050203 62.012213) (end 115.587787 62.012213) (width 0.4) (layer "F.Cu") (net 14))
 (segment (start 120 51) (end 120 47.509686) (width 0.4) (layer "F.Cu") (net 3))
 (segment (start 112.390628 52.7) (end 113.595314 51.495314) (width 0.4) (layer "F.Cu") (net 3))
 (segment (start 112.989629 52.101) (end 113.595314 51.495314) (width 0.4) (layer "F.Cu") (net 3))
 (segment (start 121.01 52.01) (end 120 51) (width 0.4) (layer "F.Cu") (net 3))
 (segment (start 120 47.509686) (end 119.499314 47.009) (width 0.4) (layer "F.Cu") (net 3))
 (segment (start 99.601 50.699) (end 100.5 49.8) (width 0.4) (layer "F.Cu") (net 3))
 (segment (start 119.499314 47.009) (end 117.079788 47.009) (width 0.4) (layer "F.Cu") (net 3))
 (segment (start 99.601 53.167914) (end 99.601 50.699) (width 0.4) (layer "F.Cu") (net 3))
 (segment (start 117.079788 47.009) (end 116.493416 47.595372) (width 0.4) (layer "F.Cu") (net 3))
 (segment (start 105.8 52.7) (end 112.390628 52.7) (width 0.4) (layer "F.Cu") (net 3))
 (segment (start 121.58 52.01) (end 121.01 52.01) (width 0.4) (layer "F.Cu") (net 3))
 (segment (start 100.5 49.8) (end 102.9 49.8) (width 0.4) (layer "F.Cu") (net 3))
 (segment (start 116.493416 47.595372) (end 116.493416 48.597213) (width 0.4) (layer "F.Cu") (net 3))
 (segment (start 100.748862 54.315776) (end 99.601 53.167914) (width 0.4) (layer "F.Cu") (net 3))
 (segment (start 102.9 49.8) (end 105.8 52.7) (width 0.4) (layer "F.Cu") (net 3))
 (segment (start 116.493416 48.597213) (end 113.595314 51.495314) (width 0.4) (layer "F.Cu") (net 3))
 (segment (start 122.74 70.46) (end 123.799 69.401) (width 0.4) (layer "F.Cu") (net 2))
 (segment (start 122.199416 70.46) (end 122.74 70.46) (width 0.4) (layer "F.Cu") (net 2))
 (segment (start 123.8 66.518477) (end 126.099 64.219477) (width 0.4) (layer "F.Cu") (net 2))
 (segment (start 126.099 64.219477) (end 126.099 57.301) (width 0.4) (layer "F.Cu") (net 2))
 (segment (start 129.208864 56.4) (end 129.8 55.808864) (width 0.4) (layer "F.Cu") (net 2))
 (segment (start 123.799 69.401) (end 123.799 66.709636) (width 0.4) (layer "F.Cu") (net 2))
 (segment (start 122.199416 69.94) (end 122.199416 70.46) (width 0.5) (layer "F.Cu") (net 2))
 (segment (start 123.8 66.708636) (end 123.8 66.518477) (width 0.4) (layer "F.Cu") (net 2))
 (segment (start 120.158416 72.501) (end 104.620416 72.501) (width 0.4) (layer "F.Cu") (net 2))
 (segment (start 129.8 50.8) (end 129 50) (width 0.4) (layer "F.Cu") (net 2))
 (segment (start 102.559416 70.61) (end 102.559416 70.44) (width 0.4) (layer "F.Cu") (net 2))
 (segment (start 123.799 66.709636) (end 123.8 66.708636) (width 0.4) (layer "F.Cu") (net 2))
 (segment (start 129.8 55.808864) (end 129.8 50.8) (width 0.4) (layer "F.Cu") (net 2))
 (segment (start 122.199416 70.46) (end 120.158416 72.501) (width 0.4) (layer "F.Cu") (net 2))
 (segment (start 104.620416 72.501) (end 102.559416 70.44) (width 0.4) (layer "F.Cu") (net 2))
 (segment (start 127 56.4) (end 129.208864 56.4) (width 0.4) (layer "F.Cu") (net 2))
 (segment (start 129 50) (end 127.6 50) (width 0.4) (layer "F.Cu") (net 2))
 (segment (start 102.659416 70.51) (end 102.559416 70.61) (width 0.4) (layer "F.Cu") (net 2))
 (segment (start 126.099 57.301) (end 127 56.4) (width 0.4) (layer "F.Cu") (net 2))
 (segment (start 118.240058 48.01) (end 118.4 48.01) (width 0.4) (layer "F.Cu") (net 7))
 (segment (start 107.209416 59.040642) (end 118.240058 48.01) (width 0.4) (layer "F.Cu") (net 7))
 (segment (start 107.209416 58.731155) (end 107.209416 59.48) (width 0.4) (layer "F.Cu") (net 7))
 (segment (start 117.769416 48.01) (end 117.769416 48.171155) (width 0.4) (layer "F.Cu") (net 7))
 (segment (start 107.209416 59.48) (end 107.209416 59.040642) (width 0.4) (layer "F.Cu") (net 7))
 (segment (start 117.09 50.01) (end 109.749416 57.350584) (width 0.4) (layer "F.Cu") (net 8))
 (segment (start 109.749416 57.350584) (end 109.749416 59.48) (width 0.4) (layer "F.Cu") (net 8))
 (segment (start 109.779416 58.25) (end 109.726186 58.30323) (width 0.2) (layer "F.Cu") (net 8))
 (segment (start 118.4 50.01) (end 117.09 50.01) (width 0.4) (layer "F.Cu") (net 8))
 (segment (start 112.299416 58.22) (end 112.290501 58.228915) (width 0.2) (layer "F.Cu") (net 9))
 (segment (start 112.289416 59.48) (end 112.289416 56.215) (width 0.4) (layer "F.Cu") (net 9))
 (segment (start 116.494416 52.01) (end 118.4 52.01) (width 0.4) (layer "F.Cu") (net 9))
 (segment (start 112.289416 56.215) (end 116.494416 52.01) (width 0.4) (layer "F.Cu") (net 9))
 (segment (start 116.19 54.01) (end 114.829416 55.370584) (width 0.4) (layer "F.Cu") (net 10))
 (segment (start 114.829416 55.370584) (end 114.829416 59.48) (width 0.4) (layer "F.Cu") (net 10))
 (segment (start 114.839416 58.27) (end 114.819416 58.29) (width 0.2) (layer "F.Cu") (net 10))
 (segment (start 116.19 54.01) (end 118.4 54.01) (width 0.4) (layer "F.Cu") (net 10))
 (segment (start 123.958 55.138909) (end 123.457 54.637909) (width 0.4) (layer "F.Cu") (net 12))
 (segment (start 123.457 49.887) (end 121.58 48.01) (width 0.4) (layer "F.Cu") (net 12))
 (segment (start 125.462416 64.006117) (end 125.462416 57.4133) (width 0.4) (layer "F.Cu") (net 12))
 (segment (start 122.199416 67.96) (end 122.199416 67.269119) (width 0.4) (layer "F.Cu") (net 12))
 (segment (start 122.199416 67.269119) (end 125.462416 64.006117) (width 0.4) (layer "F.Cu") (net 12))
 (segment (start 123.958 55.908884) (end 123.958 55.138909) (width 0.4) (layer "F.Cu") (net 12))
 (segment (start 125.462416 57.4133) (end 123.958 55.908884) (width 0.4) (layer "F.Cu") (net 12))
 (segment (start 123.457 54.637909) (end 123.457 49.887) (width 0.4) (layer "F.Cu") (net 12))
 (segment (start 122.217395 66.401196) (end 124.861416 63.757175) (width 0.4) (layer "F.Cu") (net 11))
 (segment (start 122.856 54.886851) (end 122.856 51.286) (width 0.4) (layer "F.Cu") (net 11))
 (segment (start 107.679 71.879) (end 115.921 71.879) (width 0.4) (layer "F.Cu") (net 11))
 (segment (start 122.856 51.286) (end 121.58 50.01) (width 0.4) (layer "F.Cu") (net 11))
 (segment (start 115.921 71.879) (end 121.398804 66.401196) (width 0.4) (layer "F.Cu") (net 11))
 (segment (start 103.74 67.94) (end 107.679 71.879) (width 0.4) (layer "F.Cu") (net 11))
 (segment (start 124.861416 57.662242) (end 123.357 56.157826) (width 0.4) (layer "F.Cu") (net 11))
 (segment (start 121.398804 66.401196) (end 122.217395 66.401196) (width 0.4) (layer "F.Cu") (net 11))
 (segment (start 123.357 55.387851) (end 122.856 54.886851) (width 0.4) (layer "F.Cu") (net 11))
 (segment (start 123.357 56.157826) (end 123.357 55.387851) (width 0.4) (layer "F.Cu") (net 11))
 (segment (start 124.861416 63.757175) (end 124.861416 57.662242) (width 0.4) (layer "F.Cu") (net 11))
 (segment (start 102.559416 67.94) (end 103.74 67.94) (width 0.4) (layer "F.Cu") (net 11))
 (segment (start 120.2 55.672083) (end 120.813083 55.059) (width 0.3) (layer "F.Cu") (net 13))
 (segment (start 120.2 56.8) (end 120.2 55.672083) (width 0.3) (layer "F.Cu") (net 13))
 (segment (start 118.4 58.01) (end 118.99 58.01) (width 0.3) (layer "F.Cu") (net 13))
 (segment (start 118.99 58.01) (end 120.2 56.8) (width 0.3) (layer "F.Cu") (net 13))
 (segment (start 122.806 56.386058) (end 124.310416 57.890474) (width 0.3) (layer "F.Cu") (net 13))
 (segment (start 122.806 55.616083) (end 122.806 56.386058) (width 0.3) (layer "F.Cu") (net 13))
 (segment (start 108.728 71.328) (end 107.869416 70.469416) (width 0.3) (layer "F.Cu") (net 13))
 (segment (start 107.869416 70.469416) (end 107.869416 69) (width 0.3) (layer "F.Cu") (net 13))
 (segment (start 121.170572 65.850196) (end 115.692768 71.328) (width 0.3) (layer "F.Cu") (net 13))
 (segment (start 124.310416 57.890474) (end 124.310416 63.528944) (width 0.3) (layer "F.Cu") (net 13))
 (segment (start 115.692768 71.328) (end 108.728 71.328) (width 0.3) (layer "F.Cu") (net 13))
 (segment (start 121.989164 65.850196) (end 121.170572 65.850196) (width 0.3) (layer "F.Cu") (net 13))
 (segment (start 107.869416 69.51) (end 107.869416 69) (width 0.3) (layer "F.Cu") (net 13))
 (segment (start 120.813083 55.059) (end 122.248917 55.059) (width 0.3) (layer "F.Cu") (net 13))
 (segment (start 122.248917 55.059) (end 122.806 55.616083) (width 0.3) (layer "F.Cu") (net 13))
 (segment (start 124.310416 63.528944) (end 121.989164 65.850196) (width 0.3) (layer "F.Cu") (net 13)))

